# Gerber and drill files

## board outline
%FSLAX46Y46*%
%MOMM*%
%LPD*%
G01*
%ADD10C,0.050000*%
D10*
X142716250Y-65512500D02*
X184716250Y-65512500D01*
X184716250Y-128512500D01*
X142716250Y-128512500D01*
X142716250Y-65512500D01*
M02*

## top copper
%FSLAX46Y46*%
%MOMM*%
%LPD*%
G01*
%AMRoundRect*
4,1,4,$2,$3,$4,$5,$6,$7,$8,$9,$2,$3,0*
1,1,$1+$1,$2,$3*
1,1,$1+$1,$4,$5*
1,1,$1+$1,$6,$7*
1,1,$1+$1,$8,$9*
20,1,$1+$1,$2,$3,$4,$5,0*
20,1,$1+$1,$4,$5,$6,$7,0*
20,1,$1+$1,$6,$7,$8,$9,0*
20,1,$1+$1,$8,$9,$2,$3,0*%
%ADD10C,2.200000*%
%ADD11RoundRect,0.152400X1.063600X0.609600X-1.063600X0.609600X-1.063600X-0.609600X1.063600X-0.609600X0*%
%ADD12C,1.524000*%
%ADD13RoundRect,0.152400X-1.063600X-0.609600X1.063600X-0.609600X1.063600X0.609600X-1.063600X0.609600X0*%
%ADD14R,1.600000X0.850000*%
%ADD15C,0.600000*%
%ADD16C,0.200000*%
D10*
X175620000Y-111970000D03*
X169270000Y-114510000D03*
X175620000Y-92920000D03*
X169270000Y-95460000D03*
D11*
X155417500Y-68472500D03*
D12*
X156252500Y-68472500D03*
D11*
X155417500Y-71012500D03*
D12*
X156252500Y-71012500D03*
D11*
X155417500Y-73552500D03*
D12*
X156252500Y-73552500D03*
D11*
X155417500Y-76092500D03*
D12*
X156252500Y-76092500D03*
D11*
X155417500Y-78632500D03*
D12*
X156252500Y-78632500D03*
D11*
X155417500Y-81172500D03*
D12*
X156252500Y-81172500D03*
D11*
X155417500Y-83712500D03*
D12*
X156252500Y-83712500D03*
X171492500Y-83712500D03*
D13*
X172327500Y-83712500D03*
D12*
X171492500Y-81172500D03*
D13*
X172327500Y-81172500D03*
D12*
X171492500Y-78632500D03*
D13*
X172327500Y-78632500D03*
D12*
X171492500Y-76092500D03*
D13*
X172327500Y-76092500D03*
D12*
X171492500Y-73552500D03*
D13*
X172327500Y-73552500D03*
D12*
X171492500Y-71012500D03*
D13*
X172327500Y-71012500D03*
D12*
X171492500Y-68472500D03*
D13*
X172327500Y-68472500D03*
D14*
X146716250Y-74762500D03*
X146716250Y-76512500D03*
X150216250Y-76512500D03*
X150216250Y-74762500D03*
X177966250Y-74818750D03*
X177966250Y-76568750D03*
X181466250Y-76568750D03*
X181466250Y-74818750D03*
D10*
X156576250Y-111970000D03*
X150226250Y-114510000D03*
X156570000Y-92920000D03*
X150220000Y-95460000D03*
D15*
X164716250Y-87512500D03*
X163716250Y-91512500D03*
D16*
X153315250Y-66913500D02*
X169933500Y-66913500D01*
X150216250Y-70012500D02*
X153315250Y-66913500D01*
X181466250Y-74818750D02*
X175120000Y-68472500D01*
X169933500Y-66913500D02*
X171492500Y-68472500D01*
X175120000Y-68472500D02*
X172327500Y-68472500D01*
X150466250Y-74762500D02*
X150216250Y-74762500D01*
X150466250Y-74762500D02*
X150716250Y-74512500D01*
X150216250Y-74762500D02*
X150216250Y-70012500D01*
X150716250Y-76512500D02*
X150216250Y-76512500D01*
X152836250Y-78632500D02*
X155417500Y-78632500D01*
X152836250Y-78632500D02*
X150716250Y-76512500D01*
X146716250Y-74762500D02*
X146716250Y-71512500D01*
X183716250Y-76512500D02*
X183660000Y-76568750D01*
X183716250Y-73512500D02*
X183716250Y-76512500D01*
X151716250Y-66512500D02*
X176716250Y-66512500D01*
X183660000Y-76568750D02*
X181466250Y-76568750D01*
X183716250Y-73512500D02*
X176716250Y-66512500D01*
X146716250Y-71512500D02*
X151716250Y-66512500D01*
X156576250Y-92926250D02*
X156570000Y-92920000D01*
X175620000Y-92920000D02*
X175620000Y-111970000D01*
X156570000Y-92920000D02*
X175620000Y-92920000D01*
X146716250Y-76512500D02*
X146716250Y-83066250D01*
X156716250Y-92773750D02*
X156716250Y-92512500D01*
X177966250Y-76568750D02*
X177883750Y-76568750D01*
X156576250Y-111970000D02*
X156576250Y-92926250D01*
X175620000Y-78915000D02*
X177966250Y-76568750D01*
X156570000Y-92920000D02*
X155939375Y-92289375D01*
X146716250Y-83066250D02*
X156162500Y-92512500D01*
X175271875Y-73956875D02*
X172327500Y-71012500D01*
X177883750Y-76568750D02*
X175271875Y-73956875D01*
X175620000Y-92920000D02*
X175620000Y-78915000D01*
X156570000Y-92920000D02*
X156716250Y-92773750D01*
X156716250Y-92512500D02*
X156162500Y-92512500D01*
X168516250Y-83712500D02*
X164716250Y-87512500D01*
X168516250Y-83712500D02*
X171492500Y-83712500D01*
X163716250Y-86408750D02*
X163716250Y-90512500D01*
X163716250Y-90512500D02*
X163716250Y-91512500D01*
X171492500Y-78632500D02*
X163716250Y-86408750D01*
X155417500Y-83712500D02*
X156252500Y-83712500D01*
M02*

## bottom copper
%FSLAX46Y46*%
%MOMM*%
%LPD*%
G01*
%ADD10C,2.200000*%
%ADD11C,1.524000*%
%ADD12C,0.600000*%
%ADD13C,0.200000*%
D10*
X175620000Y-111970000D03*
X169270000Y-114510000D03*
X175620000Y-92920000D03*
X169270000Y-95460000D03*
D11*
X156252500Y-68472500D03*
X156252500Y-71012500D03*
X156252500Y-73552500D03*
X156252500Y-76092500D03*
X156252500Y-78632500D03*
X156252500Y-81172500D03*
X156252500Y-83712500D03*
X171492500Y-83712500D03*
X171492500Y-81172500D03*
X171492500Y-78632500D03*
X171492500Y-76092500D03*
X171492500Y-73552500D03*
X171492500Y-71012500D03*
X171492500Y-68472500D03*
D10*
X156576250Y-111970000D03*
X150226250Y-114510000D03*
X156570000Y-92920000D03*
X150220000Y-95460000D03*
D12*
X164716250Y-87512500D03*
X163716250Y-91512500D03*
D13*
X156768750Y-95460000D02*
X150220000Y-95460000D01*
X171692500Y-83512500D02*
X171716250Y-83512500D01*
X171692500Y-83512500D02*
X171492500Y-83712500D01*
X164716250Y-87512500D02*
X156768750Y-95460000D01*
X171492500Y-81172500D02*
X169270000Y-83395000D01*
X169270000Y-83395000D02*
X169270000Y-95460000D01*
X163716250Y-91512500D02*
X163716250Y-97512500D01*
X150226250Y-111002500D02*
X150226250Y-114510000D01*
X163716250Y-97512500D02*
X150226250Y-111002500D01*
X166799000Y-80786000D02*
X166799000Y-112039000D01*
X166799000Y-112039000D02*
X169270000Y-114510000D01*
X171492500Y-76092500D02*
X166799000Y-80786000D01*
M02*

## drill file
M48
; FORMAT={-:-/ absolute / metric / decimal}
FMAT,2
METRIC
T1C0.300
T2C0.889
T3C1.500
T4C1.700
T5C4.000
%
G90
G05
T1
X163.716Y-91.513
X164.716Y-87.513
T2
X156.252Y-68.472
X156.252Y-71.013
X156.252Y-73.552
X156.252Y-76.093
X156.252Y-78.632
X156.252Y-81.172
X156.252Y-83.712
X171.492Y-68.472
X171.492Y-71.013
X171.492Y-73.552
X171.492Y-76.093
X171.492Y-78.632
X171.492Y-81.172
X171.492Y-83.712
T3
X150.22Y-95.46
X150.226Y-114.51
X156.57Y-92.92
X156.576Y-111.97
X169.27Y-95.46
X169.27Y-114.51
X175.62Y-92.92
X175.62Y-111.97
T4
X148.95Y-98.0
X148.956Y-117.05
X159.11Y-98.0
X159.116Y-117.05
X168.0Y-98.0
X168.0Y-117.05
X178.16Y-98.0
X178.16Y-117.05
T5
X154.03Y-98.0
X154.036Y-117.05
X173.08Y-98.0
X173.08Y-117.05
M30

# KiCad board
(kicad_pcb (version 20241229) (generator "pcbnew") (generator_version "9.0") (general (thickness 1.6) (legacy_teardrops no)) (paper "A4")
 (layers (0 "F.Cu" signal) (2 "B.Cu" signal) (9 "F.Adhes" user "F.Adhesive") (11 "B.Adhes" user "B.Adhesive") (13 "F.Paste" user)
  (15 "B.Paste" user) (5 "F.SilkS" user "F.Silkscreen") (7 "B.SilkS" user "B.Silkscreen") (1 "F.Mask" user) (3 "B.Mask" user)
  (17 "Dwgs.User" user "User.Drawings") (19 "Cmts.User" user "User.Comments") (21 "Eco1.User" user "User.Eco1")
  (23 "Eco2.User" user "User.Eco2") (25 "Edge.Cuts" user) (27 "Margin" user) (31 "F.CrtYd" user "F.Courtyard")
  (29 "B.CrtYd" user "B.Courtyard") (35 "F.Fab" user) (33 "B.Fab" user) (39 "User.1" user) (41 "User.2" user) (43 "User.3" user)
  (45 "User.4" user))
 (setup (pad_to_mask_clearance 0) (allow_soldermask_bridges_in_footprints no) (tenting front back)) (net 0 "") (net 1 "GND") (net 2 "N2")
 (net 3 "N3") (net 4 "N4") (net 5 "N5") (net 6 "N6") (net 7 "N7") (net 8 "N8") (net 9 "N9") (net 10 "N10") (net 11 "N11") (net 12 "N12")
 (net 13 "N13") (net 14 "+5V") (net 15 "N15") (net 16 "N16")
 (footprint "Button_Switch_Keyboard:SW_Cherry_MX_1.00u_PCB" (layer "F.Cu") (at 175.62 111.97)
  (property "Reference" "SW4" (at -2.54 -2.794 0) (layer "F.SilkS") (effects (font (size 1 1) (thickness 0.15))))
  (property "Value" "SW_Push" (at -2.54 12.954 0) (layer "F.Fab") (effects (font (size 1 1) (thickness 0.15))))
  (pad "" np_thru_hole circle (at -7.62 5.08) (size 1.7 1.7) (drill 1.7) (layers "*.Cu" "*.Mask"))
  (pad "" np_thru_hole circle (at -2.54 5.08) (size 4 4) (drill 4) (layers "*.Cu" "*.Mask"))
  (pad "" np_thru_hole circle (at 2.54 5.08) (size 1.7 1.7) (drill 1.7) (layers "*.Cu" "*.Mask"))
  (pad "1" thru_hole circle (at 0 0) (size 2.2 2.2) (drill 1.5) (layers "*.Cu" "*.Mask") (remove_unused_layers no) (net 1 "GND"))
  (pad "2" thru_hole circle (at -6.35 2.54) (size 2.2 2.2) (drill 1.5) (layers "*.Cu" "*.Mask") (remove_unused_layers no) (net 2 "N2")))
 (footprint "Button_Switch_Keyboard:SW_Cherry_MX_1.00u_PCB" (layer "F.Cu") (at 175.62 92.92)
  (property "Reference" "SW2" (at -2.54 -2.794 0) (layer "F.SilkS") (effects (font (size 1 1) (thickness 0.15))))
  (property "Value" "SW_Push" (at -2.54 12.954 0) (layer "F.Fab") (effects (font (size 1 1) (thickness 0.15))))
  (pad "" np_thru_hole circle (at -7.62 5.08) (size 1.7 1.7) (drill 1.7) (layers "*.Cu" "*.Mask"))
  (pad "" np_thru_hole circle (at -2.54 5.08) (size 4 4) (drill 4) (layers "*.Cu" "*.Mask"))
  (pad "" np_thru_hole circle (at 2.54 5.08) (size 1.7 1.7) (drill 1.7) (layers "*.Cu" "*.Mask"))
  (pad "1" thru_hole circle (at 0 0) (size 2.2 2.2) (drill 1.5) (layers "*.Cu" "*.Mask") (remove_unused_layers no) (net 1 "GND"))
  (pad "2" thru_hole circle (at -6.35 2.54) (size 2.2 2.2) (drill 1.5) (layers "*.Cu" "*.Mask") (remove_unused_layers no) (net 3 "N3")))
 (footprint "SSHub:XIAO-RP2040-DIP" (layer "F.Cu") (at 163.8725 76.0925)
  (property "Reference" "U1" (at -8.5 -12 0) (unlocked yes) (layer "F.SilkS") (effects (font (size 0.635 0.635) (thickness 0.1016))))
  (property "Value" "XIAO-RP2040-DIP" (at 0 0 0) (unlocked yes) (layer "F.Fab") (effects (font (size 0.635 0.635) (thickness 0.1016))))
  (pad "1" smd roundrect (at -8.455 -7.62 180) (size 2.432 1.524) (layers "F.Cu" "F.Mask") (roundrect_rratio 0.1) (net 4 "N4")
   (thermal_bridge_angle 45))
  (pad "1" thru_hole circle (at -7.62 -7.62 180) (size 1.524 1.524) (drill 0.889) (layers "*.Cu" "*.Mask") (remove_unused_layers no)
   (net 4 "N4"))
  (pad "2" smd roundrect (at -8.455 -5.08 180) (size 2.432 1.524) (layers "F.Cu" "F.Mask") (roundrect_rratio 0.1) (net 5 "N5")
   (thermal_bridge_angle 45))
  (pad "2" thru_hole circle (at -7.62 -5.08 180) (size 1.524 1.524) (drill 0.889) (layers "*.Cu" "*.Mask") (remove_unused_layers no)
   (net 5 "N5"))
  (pad "3" smd roundrect (at -8.455 -2.54 180) (size 2.432 1.524) (layers "F.Cu" "F.Mask") (roundrect_rratio 0.1) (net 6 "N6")
   (thermal_bridge_angle 45))
  (pad "3" thru_hole circle (at -7.62 -2.54 180) (size 1.524 1.524) (drill 0.889) (layers "*.Cu" "*.Mask") (remove_unused_layers no)
   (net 6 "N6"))
  (pad "4" smd roundrect (at -8.455 0 180) (size 2.432 1.524) (layers "F.Cu" "F.Mask") (roundrect_rratio 0.1) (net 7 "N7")
   (thermal_bridge_angle 45))
  (pad "4" thru_hole circle (at -7.62 0 180) (size 1.524 1.524) (drill 0.889) (layers "*.Cu" "*.Mask") (remove_unused_layers no)
   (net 7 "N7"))
  (pad "5" smd roundrect (at -8.455 2.54 180) (size 2.432 1.524) (layers "F.Cu" "F.Mask") (roundrect_rratio 0.1) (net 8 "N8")
   (thermal_bridge_angle 45))
  (pad "5" thru_hole circle (at -7.62 2.54 180) (size 1.524 1.524) (drill 0.889) (layers "*.Cu" "*.Mask") (remove_unused_layers no)
   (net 8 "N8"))
  (pad "6" smd roundrect (at -8.455 5.08 180) (size 2.432 1.524) (layers "F.Cu" "F.Mask") (roundrect_rratio 0.1) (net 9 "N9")
   (thermal_bridge_angle 45))
  (pad "6" thru_hole circle (at -7.62 5.08 180) (size 1.524 1.524) (drill 0.889) (layers "*.Cu" "*.Mask") (remove_unused_layers no)
   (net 9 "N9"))
  (pad "7" smd roundrect (at -8.455 7.62 180) (size 2.432 1.524) (layers "F.Cu" "F.Mask") (roundrect_rratio 0.1) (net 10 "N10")
   (thermal_bridge_angle 45))
  (pad "7" thru_hole circle (at -7.62 7.62 180) (size 1.524 1.524) (drill 0.889) (layers "*.Cu" "*.Mask") (remove_unused_layers no)
   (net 10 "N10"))
  (pad "8" thru_hole circle (at 7.62 7.62) (size 1.524 1.524) (drill 0.889) (layers "*.Cu" "*.Mask") (remove_unused_layers no)
   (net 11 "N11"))
  (pad "8" smd roundrect (at 8.455 7.62) (size 2.432 1.524) (layers "F.Cu" "F.Mask") (roundrect_rratio 0.1) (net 11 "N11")
   (thermal_bridge_angle 45))
  (pad "9" thru_hole circle (at 7.62 5.08) (size 1.524 1.524) (drill 0.889) (layers "*.Cu" "*.Mask") (remove_unused_layers no) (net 3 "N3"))
  (pad "9" smd roundrect (at 8.455 5.08) (size 2.432 1.524) (layers "F.Cu" "F.Mask") (roundrect_rratio 0.1) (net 3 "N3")
   (thermal_bridge_angle 45))
  (pad "10" thru_hole circle (at 7.62 2.54) (size 1.524 1.524) (drill 0.889) (layers "*.Cu" "*.Mask") (remove_unused_layers no)
   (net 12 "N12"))
  (pad "10" smd roundrect (at 8.455 2.54) (size 2.432 1.524) (layers "F.Cu" "F.Mask") (roundrect_rratio 0.1) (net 12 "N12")
   (thermal_bridge_angle 45))
  (pad "11" thru_hole circle (at 7.62 0) (size 1.524 1.524) (drill 0.889) (layers "*.Cu" "*.Mask") (remove_unused_layers no) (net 2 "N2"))
  (pad "11" smd roundrect (at 8.455 0) (size 2.432 1.524) (layers "F.Cu" "F.Mask") (roundrect_rratio 0.1) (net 2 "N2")
   (thermal_bridge_angle 45))
  (pad "12" thru_hole circle (at 7.62 -2.54) (size 1.524 1.524) (drill 0.889) (layers "*.Cu" "*.Mask") (remove_unused_layers no)
   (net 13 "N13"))
  (pad "12" smd roundrect (at 8.455 -2.54) (size 2.432 1.524) (layers "F.Cu" "F.Mask") (roundrect_rratio 0.1) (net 13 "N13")
   (thermal_bridge_angle 45))
  (pad "13" thru_hole circle (at 7.62 -5.08) (size 1.524 1.524) (drill 0.889) (layers "*.Cu" "*.Mask") (remove_unused_layers no)
   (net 1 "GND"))
  (pad "13" smd roundrect (at 8.455 -5.08) (size 2.432 1.524) (layers "F.Cu" "F.Mask") (roundrect_rratio 0.1) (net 1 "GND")
   (thermal_bridge_angle 45))
  (pad "14" thru_hole circle (at 7.62 -7.62) (size 1.524 1.524) (drill 0.889) (layers "*.Cu" "*.Mask") (remove_unused_layers no)
   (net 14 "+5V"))
  (pad "14" smd roundrect (at 8.455 -7.62) (size 2.432 1.524) (layers "F.Cu" "F.Mask") (roundrect_rratio 0.1) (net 14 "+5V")
   (thermal_bridge_angle 45)))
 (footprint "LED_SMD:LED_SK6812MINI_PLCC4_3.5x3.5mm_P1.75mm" (layer "F.Cu") (at 148.46625 75.6375)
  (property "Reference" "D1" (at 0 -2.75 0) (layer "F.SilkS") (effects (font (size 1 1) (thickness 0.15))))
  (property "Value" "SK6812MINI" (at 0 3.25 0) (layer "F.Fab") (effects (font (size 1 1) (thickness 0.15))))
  (pad "1" smd rect (at -1.75 -0.875) (size 1.6 0.85) (layers "F.Cu" "F.Mask" "F.Paste") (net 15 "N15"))
  (pad "2" smd rect (at -1.75 0.875) (size 1.6 0.85) (layers "F.Cu" "F.Mask" "F.Paste") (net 1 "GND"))
  (pad "3" smd rect (at 1.75 0.875) (size 1.6 0.85) (layers "F.Cu" "F.Mask" "F.Paste") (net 8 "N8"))
  (pad "4" smd rect (at 1.75 -0.875) (size 1.6 0.85) (layers "F.Cu" "F.Mask" "F.Paste") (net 14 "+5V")))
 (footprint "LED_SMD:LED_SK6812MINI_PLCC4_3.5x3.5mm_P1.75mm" (layer "F.Cu") (at 179.71625 75.69375)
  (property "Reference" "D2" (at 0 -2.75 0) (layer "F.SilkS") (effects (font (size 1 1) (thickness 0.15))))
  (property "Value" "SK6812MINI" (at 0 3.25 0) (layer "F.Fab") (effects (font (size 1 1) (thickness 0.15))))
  (pad "1" smd rect (at -1.75 -0.875) (size 1.6 0.85) (layers "F.Cu" "F.Mask" "F.Paste") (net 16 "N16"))
  (pad "2" smd rect (at -1.75 0.875) (size 1.6 0.85) (layers "F.Cu" "F.Mask" "F.Paste") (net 1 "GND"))
  (pad "3" smd rect (at 1.75 0.875) (size 1.6 0.85) (layers "F.Cu" "F.Mask" "F.Paste") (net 15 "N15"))
  (pad "4" smd rect (at 1.75 -0.875) (size 1.6 0.85) (layers "F.Cu" "F.Mask" "F.Paste") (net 14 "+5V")))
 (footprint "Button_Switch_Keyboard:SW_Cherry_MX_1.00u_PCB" (layer "F.Cu") (at 156.57625 111.97)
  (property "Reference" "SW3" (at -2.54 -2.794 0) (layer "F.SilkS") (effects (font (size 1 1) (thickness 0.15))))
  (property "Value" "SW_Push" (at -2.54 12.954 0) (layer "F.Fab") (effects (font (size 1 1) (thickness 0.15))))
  (pad "" np_thru_hole circle (at -7.62 5.08) (size 1.7 1.7) (drill 1.7) (layers "*.Cu" "*.Mask"))
  (pad "" np_thru_hole circle (at -2.54 5.08) (size 4 4) (drill 4) (layers "*.Cu" "*.Mask"))
  (pad "" np_thru_hole circle (at 2.54 5.08) (size 1.7 1.7) (drill 1.7) (layers "*.Cu" "*.Mask"))
  (pad "1" thru_hole circle (at 0 0) (size 2.2 2.2) (drill 1.5) (layers "*.Cu" "*.Mask") (remove_unused_layers no) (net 1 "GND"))
  (pad "2" thru_hole circle (at -6.35 2.54) (size 2.2 2.2) (drill 1.5) (layers "*.Cu" "*.Mask") (remove_unused_layers no) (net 12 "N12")))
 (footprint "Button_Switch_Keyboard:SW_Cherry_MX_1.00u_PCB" (layer "F.Cu") (at 156.57 92.92)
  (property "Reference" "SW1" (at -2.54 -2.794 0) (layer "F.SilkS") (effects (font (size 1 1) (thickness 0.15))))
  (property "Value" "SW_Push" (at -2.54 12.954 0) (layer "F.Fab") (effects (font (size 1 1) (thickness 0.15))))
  (pad "" np_thru_hole circle (at -7.62 5.08) (size 1.7 1.7) (drill 1.7) (layers "*.Cu" "*.Mask"))
  (pad "" np_thru_hole circle (at -2.54 5.08) (size 4 4) (drill 4) (layers "*.Cu" "*.Mask"))
  (pad "" np_thru_hole circle (at 2.54 5.08) (size 1.7 1.7) (drill 1.7) (layers "*.Cu" "*.Mask"))
  (pad "1" thru_hole circle (at 0 0) (size 2.2 2.2) (drill 1.5) (layers "*.Cu" "*.Mask") (remove_unused_layers no) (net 1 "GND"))
  (pad "2" thru_hole circle (at -6.35 2.54) (size 2.2 2.2) (drill 1.5) (layers "*.Cu" "*.Mask") (remove_unused_layers no) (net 11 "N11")))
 (gr_rect (start 142.71625 65.5125) (end 184.71625 128.5125) (stroke (width 0.05) (type default)) (fill no) (layer "Edge.Cuts"))
 (segment (start 153.31525 66.9135) (end 169.9335 66.9135) (width 0.2) (layer "F.Cu") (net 14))
 (segment (start 150.21625 70.0125) (end 153.31525 66.9135) (width 0.2) (layer "F.Cu") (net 14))
 (segment (start 181.46625 74.81875) (end 175.12 68.4725) (width 0.2) (layer "F.Cu") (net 14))
 (segment (start 169.9335 66.9135) (end 171.4925 68.4725) (width 0.2) (layer "F.Cu") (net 14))
 (segment (start 175.12 68.4725) (end 172.3275 68.4725) (width 0.2) (layer "F.Cu") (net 14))
 (segment (start 150.46625 74.7625) (end 150.21625 74.7625) (width 0.2) (layer "F.Cu") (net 14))
 (segment (start 150.46625 74.7625) (end 150.71625 74.5125) (width 0.2) (layer "F.Cu") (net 14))
 (segment (start 150.21625 74.7625) (end 150.21625 70.0125) (width 0.2) (layer "F.Cu") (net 14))
 (segment (start 150.71625 76.5125) (end 150.21625 76.5125) (width 0.2) (layer "F.Cu") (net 8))
 (segment (start 152.83625 78.6325) (end 155.4175 78.6325) (width 0.2) (layer "F.Cu") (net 8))
 (segment (start 152.83625 78.6325) (end 150.71625 76.5125) (width 0.2) (layer "F.Cu") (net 8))
 (segment (start 146.71625 74.7625) (end 146.71625 71.5125) (width 0.2) (layer "F.Cu") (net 15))
 (segment (start 183.71625 76.5125) (end 183.66 76.56875) (width 0.2) (layer "F.Cu") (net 15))
 (segment (start 183.71625 73.5125) (end 183.71625 76.5125) (width 0.2) (layer "F.Cu") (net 15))
 (segment (start 151.71625 66.5125) (end 176.71625 66.5125) (width 0.2) (layer "F.Cu") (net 15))
 (segment (start 183.66 76.56875) (end 181.46625 76.56875) (width 0.2) (layer "F.Cu") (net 15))
 (segment (start 183.71625 73.5125) (end 176.71625 66.5125) (width 0.2) (layer "F.Cu") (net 15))
 (segment (start 146.71625 71.5125) (end 151.71625 66.5125) (width 0.2) (layer "F.Cu") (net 15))
 (segment (start 156.57625 92.92625) (end 156.57 92.92) (width 0.2) (layer "F.Cu") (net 1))
 (segment (start 175.62 92.92) (end 175.62 111.97) (width 0.2) (layer "F.Cu") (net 1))
 (segment (start 156.57 92.92) (end 175.62 92.92) (width 0.2) (layer "F.Cu") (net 1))
 (segment (start 146.71625 76.5125) (end 146.71625 83.06625) (width 0.2) (layer "F.Cu") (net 1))
 (segment (start 156.71625 92.77375) (end 156.71625 92.5125) (width 0.2) (layer "F.Cu") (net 1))
 (segment (start 177.96625 76.56875) (end 177.88375 76.56875) (width 0.2) (layer "F.Cu") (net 1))
 (segment (start 156.57625 111.97) (end 156.57625 92.92625) (width 0.2) (layer "F.Cu") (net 1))
 (segment (start 175.62 78.915) (end 177.96625 76.56875) (width 0.2) (layer "F.Cu") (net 1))
 (segment (start 156.57 92.92) (end 155.939375 92.289375) (width 0.2) (layer "F.Cu") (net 1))
 (segment (start 146.71625 83.06625) (end 156.1625 92.5125) (width 0.2) (layer "F.Cu") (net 1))
 (segment (start 175.271875 73.956875) (end 172.3275 71.0125) (width 0.2) (layer "F.Cu") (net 1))
 (segment (start 177.88375 76.56875) (end 175.271875 73.956875) (width 0.2) (layer "F.Cu") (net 1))
 (segment (start 175.62 92.92) (end 175.62 78.915) (width 0.2) (layer "F.Cu") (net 1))
 (segment (start 156.57 92.92) (end 156.71625 92.77375) (width 0.2) (layer "F.Cu") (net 1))
 (segment (start 156.71625 92.5125) (end 156.1625 92.5125) (width 0.2) (layer "F.Cu") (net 1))
 (segment (start 168.51625 83.7125) (end 164.71625 87.5125) (width 0.2) (layer "F.Cu") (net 11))
 (segment (start 168.51625 83.7125) (end 171.4925 83.7125) (width 0.2) (layer "F.Cu") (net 11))
 (via (at 164.71625 87.5125) (size 0.6) (drill 0.3) (layers "F.Cu" "B.Cu") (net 11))
 (segment (start 156.76875 95.46) (end 150.22 95.46) (width 0.2) (layer "B.Cu") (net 11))
 (segment (start 171.6925 83.5125) (end 171.71625 83.5125) (width 0.2) (layer "B.Cu") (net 11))
 (segment (start 171.6925 83.5125) (end 171.4925 83.7125) (width 0.2) (layer "B.Cu") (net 11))
 (segment (start 164.71625 87.5125) (end 156.76875 95.46) (width 0.2) (layer "B.Cu") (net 11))
 (segment (start 171.4925 81.1725) (end 169.27 83.395) (width 0.2) (layer "B.Cu") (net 3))
 (segment (start 169.27 83.395) (end 169.27 95.46) (width 0.2) (layer "B.Cu") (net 3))
 (segment (start 163.71625 86.40875) (end 163.71625 90.5125) (width 0.2) (layer "F.Cu") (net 12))
 (segment (start 163.71625 90.5125) (end 163.71625 91.5125) (width 0.2) (layer "F.Cu") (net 12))
 (segment (start 171.4925 78.6325) (end 163.71625 86.40875) (width 0.2) (layer "F.Cu") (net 12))
 (via (at 163.71625 91.5125) (size 0.6) (drill 0.3) (layers "F.Cu" "B.Cu") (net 12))
 (segment (start 163.71625 91.5125) (end 163.71625 97.5125) (width 0.2) (layer "B.Cu") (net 12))
 (segment (start 150.22625 111.0025) (end 150.22625 114.51) (width 0.2) (layer "B.Cu") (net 12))
 (segment (start 163.71625 97.5125) (end 150.22625 111.0025) (width 0.2) (layer "B.Cu") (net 12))
 (segment (start 166.799 80.786) (end 166.799 112.039) (width 0.2) (layer "B.Cu") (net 2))
 (segment (start 166.799 112.039) (end 169.27 114.51) (width 0.2) (layer "B.Cu") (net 2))
 (segment (start 171.4925 76.0925) (end 166.799 80.786) (width 0.2) (layer "B.Cu") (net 2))
 (segment (start 155.4175 83.7125) (end 156.2525 83.7125) (width 0.2) (layer "F.Cu") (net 10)))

